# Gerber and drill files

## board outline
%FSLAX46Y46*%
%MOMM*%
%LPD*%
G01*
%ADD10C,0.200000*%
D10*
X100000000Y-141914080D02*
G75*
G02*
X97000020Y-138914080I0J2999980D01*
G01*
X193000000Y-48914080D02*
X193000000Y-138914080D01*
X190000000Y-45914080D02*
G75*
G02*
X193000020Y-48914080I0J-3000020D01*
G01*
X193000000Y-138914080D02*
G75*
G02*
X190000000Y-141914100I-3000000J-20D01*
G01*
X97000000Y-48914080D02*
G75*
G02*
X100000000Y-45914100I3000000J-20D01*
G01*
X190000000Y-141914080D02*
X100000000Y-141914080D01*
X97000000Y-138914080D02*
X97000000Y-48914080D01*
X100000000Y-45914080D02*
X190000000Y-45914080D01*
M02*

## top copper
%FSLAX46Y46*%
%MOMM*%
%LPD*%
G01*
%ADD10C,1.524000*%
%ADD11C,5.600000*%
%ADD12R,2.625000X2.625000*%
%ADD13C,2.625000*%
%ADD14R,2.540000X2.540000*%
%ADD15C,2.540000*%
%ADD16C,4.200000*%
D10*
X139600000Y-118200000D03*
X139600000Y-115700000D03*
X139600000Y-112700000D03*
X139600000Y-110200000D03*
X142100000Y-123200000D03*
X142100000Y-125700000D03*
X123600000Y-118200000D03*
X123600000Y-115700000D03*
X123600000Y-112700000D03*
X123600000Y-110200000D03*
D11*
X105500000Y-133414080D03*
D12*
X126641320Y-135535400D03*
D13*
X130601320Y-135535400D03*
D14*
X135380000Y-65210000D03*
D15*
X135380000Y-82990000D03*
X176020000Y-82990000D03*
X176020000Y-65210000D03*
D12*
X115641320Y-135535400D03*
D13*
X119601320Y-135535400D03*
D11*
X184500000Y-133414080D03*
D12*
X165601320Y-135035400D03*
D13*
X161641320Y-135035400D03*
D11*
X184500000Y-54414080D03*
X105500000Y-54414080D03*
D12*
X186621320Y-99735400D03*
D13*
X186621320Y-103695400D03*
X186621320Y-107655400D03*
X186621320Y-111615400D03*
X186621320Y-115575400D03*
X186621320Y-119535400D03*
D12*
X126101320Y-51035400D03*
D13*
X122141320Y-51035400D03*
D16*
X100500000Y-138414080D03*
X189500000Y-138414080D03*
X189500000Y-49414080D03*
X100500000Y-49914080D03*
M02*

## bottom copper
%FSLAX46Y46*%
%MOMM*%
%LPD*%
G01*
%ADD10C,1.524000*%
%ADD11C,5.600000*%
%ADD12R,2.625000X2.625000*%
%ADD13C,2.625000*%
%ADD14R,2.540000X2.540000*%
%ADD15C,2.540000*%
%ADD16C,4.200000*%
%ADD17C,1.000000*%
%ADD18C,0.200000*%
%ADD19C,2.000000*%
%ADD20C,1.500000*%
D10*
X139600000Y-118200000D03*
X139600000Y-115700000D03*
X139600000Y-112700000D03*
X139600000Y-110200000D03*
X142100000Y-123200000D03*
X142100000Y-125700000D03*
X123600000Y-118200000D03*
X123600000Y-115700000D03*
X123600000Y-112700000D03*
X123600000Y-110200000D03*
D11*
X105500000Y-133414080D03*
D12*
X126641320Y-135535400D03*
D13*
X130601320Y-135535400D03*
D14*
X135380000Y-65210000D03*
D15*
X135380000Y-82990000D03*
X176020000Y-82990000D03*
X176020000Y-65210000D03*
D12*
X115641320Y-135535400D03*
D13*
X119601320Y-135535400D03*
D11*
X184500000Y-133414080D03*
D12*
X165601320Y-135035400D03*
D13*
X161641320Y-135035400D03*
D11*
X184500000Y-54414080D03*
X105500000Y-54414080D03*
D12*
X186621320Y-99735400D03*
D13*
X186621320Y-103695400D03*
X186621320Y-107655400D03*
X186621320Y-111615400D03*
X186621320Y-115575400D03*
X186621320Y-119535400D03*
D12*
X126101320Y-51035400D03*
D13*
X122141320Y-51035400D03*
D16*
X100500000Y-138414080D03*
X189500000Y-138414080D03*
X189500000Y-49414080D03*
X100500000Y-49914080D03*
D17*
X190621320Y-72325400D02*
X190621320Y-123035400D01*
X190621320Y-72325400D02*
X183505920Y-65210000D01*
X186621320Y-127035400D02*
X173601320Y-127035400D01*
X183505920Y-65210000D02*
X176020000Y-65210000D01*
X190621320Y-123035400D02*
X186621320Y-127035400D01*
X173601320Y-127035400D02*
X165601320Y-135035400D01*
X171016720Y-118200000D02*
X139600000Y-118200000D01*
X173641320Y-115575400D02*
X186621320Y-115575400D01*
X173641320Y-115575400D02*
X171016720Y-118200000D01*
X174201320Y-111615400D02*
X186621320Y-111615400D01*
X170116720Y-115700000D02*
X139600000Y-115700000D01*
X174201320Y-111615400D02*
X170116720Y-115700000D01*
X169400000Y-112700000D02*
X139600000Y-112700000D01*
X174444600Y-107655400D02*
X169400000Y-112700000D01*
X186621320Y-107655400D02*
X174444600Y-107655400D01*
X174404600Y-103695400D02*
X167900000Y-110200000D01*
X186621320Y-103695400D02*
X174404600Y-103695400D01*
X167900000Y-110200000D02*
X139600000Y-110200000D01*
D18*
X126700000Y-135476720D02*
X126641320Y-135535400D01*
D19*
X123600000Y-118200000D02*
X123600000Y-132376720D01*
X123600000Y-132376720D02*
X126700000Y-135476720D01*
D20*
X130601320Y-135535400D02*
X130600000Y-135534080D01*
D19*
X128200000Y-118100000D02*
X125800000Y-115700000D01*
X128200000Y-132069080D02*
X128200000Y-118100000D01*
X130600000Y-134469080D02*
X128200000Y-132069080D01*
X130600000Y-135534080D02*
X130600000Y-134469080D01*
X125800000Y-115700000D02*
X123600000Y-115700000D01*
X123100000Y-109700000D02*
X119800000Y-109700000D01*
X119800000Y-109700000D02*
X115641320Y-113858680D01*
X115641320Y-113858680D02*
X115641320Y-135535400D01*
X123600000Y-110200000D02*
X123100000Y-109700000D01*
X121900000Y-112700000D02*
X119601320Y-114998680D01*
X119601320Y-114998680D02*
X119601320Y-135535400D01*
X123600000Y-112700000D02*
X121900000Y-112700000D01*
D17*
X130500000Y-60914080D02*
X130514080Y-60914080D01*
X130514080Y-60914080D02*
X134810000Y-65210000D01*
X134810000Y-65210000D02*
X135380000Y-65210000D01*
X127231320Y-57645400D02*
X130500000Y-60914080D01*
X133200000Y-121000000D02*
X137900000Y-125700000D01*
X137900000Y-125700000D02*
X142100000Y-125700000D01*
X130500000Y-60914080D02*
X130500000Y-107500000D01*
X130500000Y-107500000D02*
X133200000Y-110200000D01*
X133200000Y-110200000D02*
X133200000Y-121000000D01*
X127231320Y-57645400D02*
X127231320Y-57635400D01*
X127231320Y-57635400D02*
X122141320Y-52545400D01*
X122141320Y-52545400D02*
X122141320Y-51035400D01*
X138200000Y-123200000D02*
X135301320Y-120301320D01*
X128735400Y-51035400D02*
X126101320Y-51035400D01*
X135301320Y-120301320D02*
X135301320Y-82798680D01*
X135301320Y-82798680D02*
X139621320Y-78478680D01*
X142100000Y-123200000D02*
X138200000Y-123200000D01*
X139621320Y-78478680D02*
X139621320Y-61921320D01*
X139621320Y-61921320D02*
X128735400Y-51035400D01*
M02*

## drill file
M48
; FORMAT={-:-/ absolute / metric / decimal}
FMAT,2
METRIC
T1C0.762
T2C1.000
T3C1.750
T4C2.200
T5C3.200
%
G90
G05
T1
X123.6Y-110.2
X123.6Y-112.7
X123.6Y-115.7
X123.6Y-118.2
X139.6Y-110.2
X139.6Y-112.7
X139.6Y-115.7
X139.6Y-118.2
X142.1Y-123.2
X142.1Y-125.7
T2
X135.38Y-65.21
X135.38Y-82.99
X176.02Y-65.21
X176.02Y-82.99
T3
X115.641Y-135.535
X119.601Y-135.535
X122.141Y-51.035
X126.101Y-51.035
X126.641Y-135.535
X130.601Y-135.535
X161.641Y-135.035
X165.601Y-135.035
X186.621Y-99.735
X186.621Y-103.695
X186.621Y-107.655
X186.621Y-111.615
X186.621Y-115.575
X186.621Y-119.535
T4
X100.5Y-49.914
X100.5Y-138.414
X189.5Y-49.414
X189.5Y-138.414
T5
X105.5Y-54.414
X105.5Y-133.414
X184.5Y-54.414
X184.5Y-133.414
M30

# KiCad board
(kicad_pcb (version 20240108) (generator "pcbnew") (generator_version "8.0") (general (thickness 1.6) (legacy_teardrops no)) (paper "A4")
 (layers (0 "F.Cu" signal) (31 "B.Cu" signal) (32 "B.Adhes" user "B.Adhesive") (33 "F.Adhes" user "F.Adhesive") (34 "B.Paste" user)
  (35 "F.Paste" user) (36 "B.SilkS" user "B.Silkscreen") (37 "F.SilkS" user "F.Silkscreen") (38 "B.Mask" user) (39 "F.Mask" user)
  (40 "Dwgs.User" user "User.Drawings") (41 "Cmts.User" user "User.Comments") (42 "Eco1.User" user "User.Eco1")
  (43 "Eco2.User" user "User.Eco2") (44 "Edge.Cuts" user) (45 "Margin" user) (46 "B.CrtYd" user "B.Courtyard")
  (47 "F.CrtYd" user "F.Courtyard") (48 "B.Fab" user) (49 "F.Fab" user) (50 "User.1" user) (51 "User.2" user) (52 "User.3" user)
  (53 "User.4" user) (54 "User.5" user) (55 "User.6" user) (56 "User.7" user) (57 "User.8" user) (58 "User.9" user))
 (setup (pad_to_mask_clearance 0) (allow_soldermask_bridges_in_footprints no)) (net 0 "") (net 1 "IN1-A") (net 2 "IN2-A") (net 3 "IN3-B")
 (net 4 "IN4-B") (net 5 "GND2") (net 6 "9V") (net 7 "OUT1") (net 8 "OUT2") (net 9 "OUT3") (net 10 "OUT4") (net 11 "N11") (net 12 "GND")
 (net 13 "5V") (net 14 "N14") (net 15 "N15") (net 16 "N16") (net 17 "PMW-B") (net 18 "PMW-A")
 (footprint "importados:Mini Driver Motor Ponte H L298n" (layer "F.Cu") (at 132.1 137.2 180)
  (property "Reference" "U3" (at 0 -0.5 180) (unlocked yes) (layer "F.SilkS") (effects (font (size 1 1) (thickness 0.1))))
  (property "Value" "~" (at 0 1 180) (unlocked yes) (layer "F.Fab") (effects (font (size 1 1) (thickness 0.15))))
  (pad "1" thru_hole circle (at -7.5 19 180) (size 1.524 1.524) (drill 0.762) (layers "*.Cu" "*.Mask") (remove_unused_layers no)
   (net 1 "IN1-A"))
  (pad "2" thru_hole circle (at -7.5 21.5 180) (size 1.524 1.524) (drill 0.762) (layers "*.Cu" "*.Mask") (remove_unused_layers no)
   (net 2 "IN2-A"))
  (pad "3" thru_hole circle (at -7.5 24.5 180) (size 1.524 1.524) (drill 0.762) (layers "*.Cu" "*.Mask") (remove_unused_layers no)
   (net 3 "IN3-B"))
  (pad "4" thru_hole circle (at -7.5 27 180) (size 1.524 1.524) (drill 0.762) (layers "*.Cu" "*.Mask") (remove_unused_layers no)
   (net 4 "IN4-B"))
  (pad "5" thru_hole circle (at -10 14 180) (size 1.524 1.524) (drill 0.762) (layers "*.Cu" "*.Mask") (remove_unused_layers no)
   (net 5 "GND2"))
  (pad "6" thru_hole circle (at -10 11.5 180) (size 1.524 1.524) (drill 0.762) (layers "*.Cu" "*.Mask") (remove_unused_layers no)
   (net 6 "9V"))
  (pad "7" thru_hole circle (at 8.5 19 180) (size 1.524 1.524) (drill 0.762) (layers "*.Cu" "*.Mask") (remove_unused_layers no)
   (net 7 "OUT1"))
  (pad "8" thru_hole circle (at 8.5 21.5 180) (size 1.524 1.524) (drill 0.762) (layers "*.Cu" "*.Mask") (remove_unused_layers no)
   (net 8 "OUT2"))
  (pad "9" thru_hole circle (at 8.5 24.5 180) (size 1.524 1.524) (drill 0.762) (layers "*.Cu" "*.Mask") (remove_unused_layers no)
   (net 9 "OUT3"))
  (pad "10" thru_hole circle (at 8.5 27 180) (size 1.524 1.524) (drill 0.762) (layers "*.Cu" "*.Mask") (remove_unused_layers no)
   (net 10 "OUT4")))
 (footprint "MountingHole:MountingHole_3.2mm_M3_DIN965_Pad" (layer "F.Cu") (at 105.5 133.41408)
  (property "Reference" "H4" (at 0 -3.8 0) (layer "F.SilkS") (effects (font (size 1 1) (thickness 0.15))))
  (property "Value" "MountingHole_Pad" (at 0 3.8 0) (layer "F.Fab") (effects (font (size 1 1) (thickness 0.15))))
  (pad "1" thru_hole circle (at 0 0) (size 5.6 5.6) (drill 3.2) (layers "*.Cu" "*.Mask") (remove_unused_layers no) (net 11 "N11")))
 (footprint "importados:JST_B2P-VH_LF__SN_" (layer "F.Cu") (at 128.62132 135.5354)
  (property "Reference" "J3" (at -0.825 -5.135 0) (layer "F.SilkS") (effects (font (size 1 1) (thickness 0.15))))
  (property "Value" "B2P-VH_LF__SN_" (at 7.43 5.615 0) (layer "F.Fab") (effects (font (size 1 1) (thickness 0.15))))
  (pad "1" thru_hole rect (at -1.98 0) (size 2.625 2.625) (drill 1.75) (layers "*.Cu" "*.Mask") (remove_unused_layers no) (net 7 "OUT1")
   (solder_mask_margin 0.102))
  (pad "2" thru_hole circle (at 1.98 0) (size 2.625 2.625) (drill 1.75) (layers "*.Cu" "*.Mask") (remove_unused_layers no) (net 8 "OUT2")
   (solder_mask_margin 0.102)))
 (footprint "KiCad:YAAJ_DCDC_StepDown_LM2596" (layer "F.Cu") (at 135.38 65.21)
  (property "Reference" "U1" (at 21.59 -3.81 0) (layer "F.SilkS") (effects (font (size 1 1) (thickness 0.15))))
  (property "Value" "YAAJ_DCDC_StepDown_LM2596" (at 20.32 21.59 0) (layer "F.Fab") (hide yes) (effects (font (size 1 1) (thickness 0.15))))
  (pad "1" thru_hole rect (at 0 0) (size 2.54 2.54) (drill 1) (layers "*.Cu" "*.Mask") (remove_unused_layers no) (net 6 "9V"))
  (pad "2" thru_hole circle (at 0 17.78) (size 2.54 2.54) (drill 1) (layers "*.Cu" "*.Mask") (remove_unused_layers no) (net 5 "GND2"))
  (pad "3" thru_hole circle (at 40.64 17.78) (size 2.54 2.54) (drill 1) (layers "*.Cu" "*.Mask") (remove_unused_layers no) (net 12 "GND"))
  (pad "4" thru_hole circle (at 40.64 0) (size 2.54 2.54) (drill 1) (layers "*.Cu" "*.Mask") (remove_unused_layers no) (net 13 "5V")))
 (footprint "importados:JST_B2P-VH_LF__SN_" (layer "F.Cu") (at 117.62132 135.5354)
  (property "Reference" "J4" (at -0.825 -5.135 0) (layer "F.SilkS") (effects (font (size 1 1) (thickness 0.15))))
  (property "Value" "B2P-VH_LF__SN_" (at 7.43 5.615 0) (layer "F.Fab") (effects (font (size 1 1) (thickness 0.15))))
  (pad "1" thru_hole rect (at -1.98 0) (size 2.625 2.625) (drill 1.75) (layers "*.Cu" "*.Mask") (remove_unused_layers no) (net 10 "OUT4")
   (solder_mask_margin 0.102))
  (pad "2" thru_hole circle (at 1.98 0) (size 2.625 2.625) (drill 1.75) (layers "*.Cu" "*.Mask") (remove_unused_layers no) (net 9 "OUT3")
   (solder_mask_margin 0.102)))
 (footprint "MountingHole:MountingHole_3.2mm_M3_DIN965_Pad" (layer "F.Cu") (at 184.5 133.41408)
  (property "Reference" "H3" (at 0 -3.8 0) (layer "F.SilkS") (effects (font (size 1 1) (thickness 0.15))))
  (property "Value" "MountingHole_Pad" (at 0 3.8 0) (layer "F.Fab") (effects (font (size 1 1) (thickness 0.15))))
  (pad "1" thru_hole circle (at 0 0) (size 5.6 5.6) (drill 3.2) (layers "*.Cu" "*.Mask") (remove_unused_layers no) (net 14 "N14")))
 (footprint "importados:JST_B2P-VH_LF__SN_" (layer "F.Cu") (at 163.62132 135.0354 180)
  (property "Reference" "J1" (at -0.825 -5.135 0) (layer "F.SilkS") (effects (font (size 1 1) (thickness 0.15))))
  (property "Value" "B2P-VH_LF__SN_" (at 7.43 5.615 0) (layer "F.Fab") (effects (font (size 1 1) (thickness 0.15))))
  (pad "1" thru_hole rect (at -1.98 0 180) (size 2.625 2.625) (drill 1.75) (layers "*.Cu" "*.Mask") (remove_unused_layers no) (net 13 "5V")
   (solder_mask_margin 0.102))
  (pad "2" thru_hole circle (at 1.98 0 180) (size 2.625 2.625) (drill 1.75) (layers "*.Cu" "*.Mask") (remove_unused_layers no)
   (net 12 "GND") (solder_mask_margin 0.102)))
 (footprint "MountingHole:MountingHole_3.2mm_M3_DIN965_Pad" (layer "F.Cu") (at 184.5 54.41408)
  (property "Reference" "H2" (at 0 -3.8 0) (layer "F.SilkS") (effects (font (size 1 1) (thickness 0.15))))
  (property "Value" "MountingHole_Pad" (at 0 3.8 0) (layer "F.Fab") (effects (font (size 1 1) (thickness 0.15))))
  (pad "1" thru_hole circle (at 0 0) (size 5.6 5.6) (drill 3.2) (layers "*.Cu" "*.Mask") (remove_unused_layers no) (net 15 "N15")))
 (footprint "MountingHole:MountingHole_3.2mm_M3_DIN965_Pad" (layer "F.Cu") (at 105.5 54.41408)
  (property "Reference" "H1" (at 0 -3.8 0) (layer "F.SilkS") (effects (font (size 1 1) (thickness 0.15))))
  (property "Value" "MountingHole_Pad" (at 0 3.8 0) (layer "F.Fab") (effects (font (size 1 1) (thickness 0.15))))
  (pad "1" thru_hole circle (at 0 0) (size 5.6 5.6) (drill 3.2) (layers "*.Cu" "*.Mask") (remove_unused_layers no) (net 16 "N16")))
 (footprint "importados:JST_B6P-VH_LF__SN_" (layer "F.Cu") (at 186.62132 109.6354 -90)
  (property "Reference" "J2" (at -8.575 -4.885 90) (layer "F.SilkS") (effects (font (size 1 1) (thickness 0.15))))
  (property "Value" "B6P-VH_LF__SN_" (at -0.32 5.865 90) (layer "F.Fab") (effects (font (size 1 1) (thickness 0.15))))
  (pad "1" thru_hole rect (at -9.9 0 270) (size 2.625 2.625) (drill 1.75) (layers "*.Cu" "*.Mask") (remove_unused_layers no)
   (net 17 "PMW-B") (solder_mask_margin 0.102))
  (pad "2" thru_hole circle (at -5.94 0 270) (size 2.625 2.625) (drill 1.75) (layers "*.Cu" "*.Mask") (remove_unused_layers no)
   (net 4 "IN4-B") (solder_mask_margin 0.102))
  (pad "3" thru_hole circle (at -1.98 0 270) (size 2.625 2.625) (drill 1.75) (layers "*.Cu" "*.Mask") (remove_unused_layers no)
   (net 3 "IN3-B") (solder_mask_margin 0.102))
  (pad "4" thru_hole circle (at 1.98 0 270) (size 2.625 2.625) (drill 1.75) (layers "*.Cu" "*.Mask") (remove_unused_layers no)
   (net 2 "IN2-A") (solder_mask_margin 0.102))
  (pad "5" thru_hole circle (at 5.94 0 270) (size 2.625 2.625) (drill 1.75) (layers "*.Cu" "*.Mask") (remove_unused_layers no)
   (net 1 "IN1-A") (solder_mask_margin 0.102))
  (pad "6" thru_hole circle (at 9.9 0 270) (size 2.625 2.625) (drill 1.75) (layers "*.Cu" "*.Mask") (remove_unused_layers no)
   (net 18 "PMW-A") (solder_mask_margin 0.102)))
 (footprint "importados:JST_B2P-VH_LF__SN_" (layer "F.Cu") (at 124.12132 51.0354 180)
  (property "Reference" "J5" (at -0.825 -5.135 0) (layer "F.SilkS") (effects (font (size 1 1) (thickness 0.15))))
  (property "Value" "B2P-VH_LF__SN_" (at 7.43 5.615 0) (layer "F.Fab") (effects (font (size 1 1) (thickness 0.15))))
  (pad "1" thru_hole rect (at -1.98 0 180) (size 2.625 2.625) (drill 1.75) (layers "*.Cu" "*.Mask") (remove_unused_layers no) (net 5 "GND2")
   (solder_mask_margin 0.102))
  (pad "2" thru_hole circle (at 1.98 0 180) (size 2.625 2.625) (drill 1.75) (layers "*.Cu" "*.Mask") (remove_unused_layers no) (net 6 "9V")
   (solder_mask_margin 0.102)))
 (gr_arc (start 100 141.91408) (mid 97.878664 141.035398) (end 97 138.91408) (stroke (width 0.2) (type default)) (layer "Edge.Cuts"))
 (gr_line (start 193 48.91408) (end 193 138.91408) (stroke (width 0.2) (type default)) (layer "Edge.Cuts"))
 (gr_arc (start 190 45.91408) (mid 192.121305 46.792757) (end 193 48.91408) (stroke (width 0.2) (type default)) (layer "Edge.Cuts"))
 (gr_arc (start 193 138.91408) (mid 192.121326 141.035406) (end 190 141.91408) (stroke (width 0.2) (type default)) (layer "Edge.Cuts"))
 (gr_arc (start 97 48.91408) (mid 97.878686 46.792766) (end 100 45.91408) (stroke (width 0.2) (type default)) (layer "Edge.Cuts"))
 (gr_line (start 190 141.91408) (end 100 141.91408) (stroke (width 0.2) (type default)) (layer "Edge.Cuts"))
 (gr_line (start 97 138.91408) (end 97 48.91408) (stroke (width 0.2) (type default)) (layer "Edge.Cuts"))
 (gr_line (start 100 45.91408) (end 190 45.91408) (stroke (width 0.2) (type default)) (layer "Edge.Cuts"))
 (via (at 100.5 138.41408) (size 4.2) (drill 2.2) (layers "F.Cu" "B.Cu") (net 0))
 (via (at 189.5 138.41408) (size 4.2) (drill 2.2) (layers "F.Cu" "B.Cu") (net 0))
 (via (at 189.5 49.41408) (size 4.2) (drill 2.2) (layers "F.Cu" "B.Cu") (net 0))
 (via (at 100.5 49.91408) (size 4.2) (drill 2.2) (layers "F.Cu" "B.Cu") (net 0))
 (segment (start 190.62132 72.3254) (end 190.62132 123.0354) (width 1) (layer "B.Cu") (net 13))
 (segment (start 190.62132 72.3254) (end 183.50592 65.21) (width 1) (layer "B.Cu") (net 13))
 (segment (start 186.62132 127.0354) (end 173.60132 127.0354) (width 1) (layer "B.Cu") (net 13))
 (segment (start 183.50592 65.21) (end 176.02 65.21) (width 1) (layer "B.Cu") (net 13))
 (segment (start 190.62132 123.0354) (end 186.62132 127.0354) (width 1) (layer "B.Cu") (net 13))
 (segment (start 173.60132 127.0354) (end 165.60132 135.0354) (width 1) (layer "B.Cu") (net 13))
 (segment (start 171.01672 118.2) (end 139.6 118.2) (width 1) (layer "B.Cu") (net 1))
 (segment (start 173.64132 115.5754) (end 186.62132 115.5754) (width 1) (layer "B.Cu") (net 1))
 (segment (start 173.64132 115.5754) (end 171.01672 118.2) (width 1) (layer "B.Cu") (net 1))
 (segment (start 174.20132 111.6154) (end 186.62132 111.6154) (width 1) (layer "B.Cu") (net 2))
 (segment (start 170.11672 115.7) (end 139.6 115.7) (width 1) (layer "B.Cu") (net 2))
 (segment (start 174.20132 111.6154) (end 170.11672 115.7) (width 1) (layer "B.Cu") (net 2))
 (segment (start 169.4 112.7) (end 139.6 112.7) (width 1) (layer "B.Cu") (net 3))
 (segment (start 174.4446 107.6554) (end 169.4 112.7) (width 1) (layer "B.Cu") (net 3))
 (segment (start 186.62132 107.6554) (end 174.4446 107.6554) (width 1) (layer "B.Cu") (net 3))
 (segment (start 174.4046 103.6954) (end 167.9 110.2) (width 1) (layer "B.Cu") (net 4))
 (segment (start 186.62132 103.6954) (end 174.4046 103.6954) (width 1) (layer "B.Cu") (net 4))
 (segment (start 167.9 110.2) (end 139.6 110.2) (width 1) (layer "B.Cu") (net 4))
 (segment (start 126.7 135.47672) (end 126.64132 135.5354) (width 0.2) (layer "B.Cu") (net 7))
 (segment (start 123.6 118.2) (end 123.6 132.37672) (width 2) (layer "B.Cu") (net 7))
 (segment (start 123.6 132.37672) (end 126.7 135.47672) (width 2) (layer "B.Cu") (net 7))
 (segment (start 130.60132 135.5354) (end 130.6 135.53408) (width 1.5) (layer "B.Cu") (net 8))
 (segment (start 128.2 118.1) (end 125.8 115.7) (width 2) (layer "B.Cu") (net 8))
 (segment (start 128.2 132.06908) (end 128.2 118.1) (width 2) (layer "B.Cu") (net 8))
 (segment (start 130.6 134.46908) (end 128.2 132.06908) (width 2) (layer "B.Cu") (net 8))
 (segment (start 130.6 135.53408) (end 130.6 134.46908) (width 2) (layer "B.Cu") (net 8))
 (segment (start 125.8 115.7) (end 123.6 115.7) (width 2) (layer "B.Cu") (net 8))
 (segment (start 123.1 109.7) (end 119.8 109.7) (width 2) (layer "B.Cu") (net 10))
 (segment (start 119.8 109.7) (end 115.64132 113.85868) (width 2) (layer "B.Cu") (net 10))
 (segment (start 115.64132 113.85868) (end 115.64132 135.5354) (width 2) (layer "B.Cu") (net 10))
 (segment (start 123.6 110.2) (end 123.1 109.7) (width 2) (layer "B.Cu") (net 10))
 (segment (start 121.9 112.7) (end 119.60132 114.99868) (width 2) (layer "B.Cu") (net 9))
 (segment (start 119.60132 114.99868) (end 119.60132 135.5354) (width 2) (layer "B.Cu") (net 9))
 (segment (start 123.6 112.7) (end 121.9 112.7) (width 2) (layer "B.Cu") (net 9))
 (segment (start 130.5 60.91408) (end 130.51408 60.91408) (width 1) (layer "B.Cu") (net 6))
 (segment (start 130.51408 60.91408) (end 134.81 65.21) (width 1) (layer "B.Cu") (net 6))
 (segment (start 134.81 65.21) (end 135.38 65.21) (width 1) (layer "B.Cu") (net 6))
 (segment (start 127.23132 57.6454) (end 130.5 60.91408) (width 1) (layer "B.Cu") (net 6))
 (segment (start 133.2 121) (end 137.9 125.7) (width 1) (layer "B.Cu") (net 6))
 (segment (start 137.9 125.7) (end 142.1 125.7) (width 1) (layer "B.Cu") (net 6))
 (segment (start 130.5 60.91408) (end 130.5 107.5) (width 1) (layer "B.Cu") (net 6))
 (segment (start 130.5 107.5) (end 133.2 110.2) (width 1) (layer "B.Cu") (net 6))
 (segment (start 133.2 110.2) (end 133.2 121) (width 1) (layer "B.Cu") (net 6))
 (segment (start 127.23132 57.6454) (end 127.23132 57.6354) (width 1) (layer "B.Cu") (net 6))
 (segment (start 127.23132 57.6354) (end 122.14132 52.5454) (width 1) (layer "B.Cu") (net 6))
 (segment (start 122.14132 52.5454) (end 122.14132 51.0354) (width 1) (layer "B.Cu") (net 6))
 (segment (start 138.2 123.2) (end 135.30132 120.30132) (width 1) (layer "B.Cu") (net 5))
 (segment (start 128.7354 51.0354) (end 126.10132 51.0354) (width 1) (layer "B.Cu") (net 5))
 (segment (start 135.30132 120.30132) (end 135.30132 82.79868) (width 1) (layer "B.Cu") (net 5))
 (segment (start 135.30132 82.79868) (end 139.62132 78.47868) (width 1) (layer "B.Cu") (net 5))
 (segment (start 142.1 123.2) (end 138.2 123.2) (width 1) (layer "B.Cu") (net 5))
 (segment (start 139.62132 78.47868) (end 139.62132 61.92132) (width 1) (layer "B.Cu") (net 5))
 (segment (start 139.62132 61.92132) (end 128.7354 51.0354) (width 1) (layer "B.Cu") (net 5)))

